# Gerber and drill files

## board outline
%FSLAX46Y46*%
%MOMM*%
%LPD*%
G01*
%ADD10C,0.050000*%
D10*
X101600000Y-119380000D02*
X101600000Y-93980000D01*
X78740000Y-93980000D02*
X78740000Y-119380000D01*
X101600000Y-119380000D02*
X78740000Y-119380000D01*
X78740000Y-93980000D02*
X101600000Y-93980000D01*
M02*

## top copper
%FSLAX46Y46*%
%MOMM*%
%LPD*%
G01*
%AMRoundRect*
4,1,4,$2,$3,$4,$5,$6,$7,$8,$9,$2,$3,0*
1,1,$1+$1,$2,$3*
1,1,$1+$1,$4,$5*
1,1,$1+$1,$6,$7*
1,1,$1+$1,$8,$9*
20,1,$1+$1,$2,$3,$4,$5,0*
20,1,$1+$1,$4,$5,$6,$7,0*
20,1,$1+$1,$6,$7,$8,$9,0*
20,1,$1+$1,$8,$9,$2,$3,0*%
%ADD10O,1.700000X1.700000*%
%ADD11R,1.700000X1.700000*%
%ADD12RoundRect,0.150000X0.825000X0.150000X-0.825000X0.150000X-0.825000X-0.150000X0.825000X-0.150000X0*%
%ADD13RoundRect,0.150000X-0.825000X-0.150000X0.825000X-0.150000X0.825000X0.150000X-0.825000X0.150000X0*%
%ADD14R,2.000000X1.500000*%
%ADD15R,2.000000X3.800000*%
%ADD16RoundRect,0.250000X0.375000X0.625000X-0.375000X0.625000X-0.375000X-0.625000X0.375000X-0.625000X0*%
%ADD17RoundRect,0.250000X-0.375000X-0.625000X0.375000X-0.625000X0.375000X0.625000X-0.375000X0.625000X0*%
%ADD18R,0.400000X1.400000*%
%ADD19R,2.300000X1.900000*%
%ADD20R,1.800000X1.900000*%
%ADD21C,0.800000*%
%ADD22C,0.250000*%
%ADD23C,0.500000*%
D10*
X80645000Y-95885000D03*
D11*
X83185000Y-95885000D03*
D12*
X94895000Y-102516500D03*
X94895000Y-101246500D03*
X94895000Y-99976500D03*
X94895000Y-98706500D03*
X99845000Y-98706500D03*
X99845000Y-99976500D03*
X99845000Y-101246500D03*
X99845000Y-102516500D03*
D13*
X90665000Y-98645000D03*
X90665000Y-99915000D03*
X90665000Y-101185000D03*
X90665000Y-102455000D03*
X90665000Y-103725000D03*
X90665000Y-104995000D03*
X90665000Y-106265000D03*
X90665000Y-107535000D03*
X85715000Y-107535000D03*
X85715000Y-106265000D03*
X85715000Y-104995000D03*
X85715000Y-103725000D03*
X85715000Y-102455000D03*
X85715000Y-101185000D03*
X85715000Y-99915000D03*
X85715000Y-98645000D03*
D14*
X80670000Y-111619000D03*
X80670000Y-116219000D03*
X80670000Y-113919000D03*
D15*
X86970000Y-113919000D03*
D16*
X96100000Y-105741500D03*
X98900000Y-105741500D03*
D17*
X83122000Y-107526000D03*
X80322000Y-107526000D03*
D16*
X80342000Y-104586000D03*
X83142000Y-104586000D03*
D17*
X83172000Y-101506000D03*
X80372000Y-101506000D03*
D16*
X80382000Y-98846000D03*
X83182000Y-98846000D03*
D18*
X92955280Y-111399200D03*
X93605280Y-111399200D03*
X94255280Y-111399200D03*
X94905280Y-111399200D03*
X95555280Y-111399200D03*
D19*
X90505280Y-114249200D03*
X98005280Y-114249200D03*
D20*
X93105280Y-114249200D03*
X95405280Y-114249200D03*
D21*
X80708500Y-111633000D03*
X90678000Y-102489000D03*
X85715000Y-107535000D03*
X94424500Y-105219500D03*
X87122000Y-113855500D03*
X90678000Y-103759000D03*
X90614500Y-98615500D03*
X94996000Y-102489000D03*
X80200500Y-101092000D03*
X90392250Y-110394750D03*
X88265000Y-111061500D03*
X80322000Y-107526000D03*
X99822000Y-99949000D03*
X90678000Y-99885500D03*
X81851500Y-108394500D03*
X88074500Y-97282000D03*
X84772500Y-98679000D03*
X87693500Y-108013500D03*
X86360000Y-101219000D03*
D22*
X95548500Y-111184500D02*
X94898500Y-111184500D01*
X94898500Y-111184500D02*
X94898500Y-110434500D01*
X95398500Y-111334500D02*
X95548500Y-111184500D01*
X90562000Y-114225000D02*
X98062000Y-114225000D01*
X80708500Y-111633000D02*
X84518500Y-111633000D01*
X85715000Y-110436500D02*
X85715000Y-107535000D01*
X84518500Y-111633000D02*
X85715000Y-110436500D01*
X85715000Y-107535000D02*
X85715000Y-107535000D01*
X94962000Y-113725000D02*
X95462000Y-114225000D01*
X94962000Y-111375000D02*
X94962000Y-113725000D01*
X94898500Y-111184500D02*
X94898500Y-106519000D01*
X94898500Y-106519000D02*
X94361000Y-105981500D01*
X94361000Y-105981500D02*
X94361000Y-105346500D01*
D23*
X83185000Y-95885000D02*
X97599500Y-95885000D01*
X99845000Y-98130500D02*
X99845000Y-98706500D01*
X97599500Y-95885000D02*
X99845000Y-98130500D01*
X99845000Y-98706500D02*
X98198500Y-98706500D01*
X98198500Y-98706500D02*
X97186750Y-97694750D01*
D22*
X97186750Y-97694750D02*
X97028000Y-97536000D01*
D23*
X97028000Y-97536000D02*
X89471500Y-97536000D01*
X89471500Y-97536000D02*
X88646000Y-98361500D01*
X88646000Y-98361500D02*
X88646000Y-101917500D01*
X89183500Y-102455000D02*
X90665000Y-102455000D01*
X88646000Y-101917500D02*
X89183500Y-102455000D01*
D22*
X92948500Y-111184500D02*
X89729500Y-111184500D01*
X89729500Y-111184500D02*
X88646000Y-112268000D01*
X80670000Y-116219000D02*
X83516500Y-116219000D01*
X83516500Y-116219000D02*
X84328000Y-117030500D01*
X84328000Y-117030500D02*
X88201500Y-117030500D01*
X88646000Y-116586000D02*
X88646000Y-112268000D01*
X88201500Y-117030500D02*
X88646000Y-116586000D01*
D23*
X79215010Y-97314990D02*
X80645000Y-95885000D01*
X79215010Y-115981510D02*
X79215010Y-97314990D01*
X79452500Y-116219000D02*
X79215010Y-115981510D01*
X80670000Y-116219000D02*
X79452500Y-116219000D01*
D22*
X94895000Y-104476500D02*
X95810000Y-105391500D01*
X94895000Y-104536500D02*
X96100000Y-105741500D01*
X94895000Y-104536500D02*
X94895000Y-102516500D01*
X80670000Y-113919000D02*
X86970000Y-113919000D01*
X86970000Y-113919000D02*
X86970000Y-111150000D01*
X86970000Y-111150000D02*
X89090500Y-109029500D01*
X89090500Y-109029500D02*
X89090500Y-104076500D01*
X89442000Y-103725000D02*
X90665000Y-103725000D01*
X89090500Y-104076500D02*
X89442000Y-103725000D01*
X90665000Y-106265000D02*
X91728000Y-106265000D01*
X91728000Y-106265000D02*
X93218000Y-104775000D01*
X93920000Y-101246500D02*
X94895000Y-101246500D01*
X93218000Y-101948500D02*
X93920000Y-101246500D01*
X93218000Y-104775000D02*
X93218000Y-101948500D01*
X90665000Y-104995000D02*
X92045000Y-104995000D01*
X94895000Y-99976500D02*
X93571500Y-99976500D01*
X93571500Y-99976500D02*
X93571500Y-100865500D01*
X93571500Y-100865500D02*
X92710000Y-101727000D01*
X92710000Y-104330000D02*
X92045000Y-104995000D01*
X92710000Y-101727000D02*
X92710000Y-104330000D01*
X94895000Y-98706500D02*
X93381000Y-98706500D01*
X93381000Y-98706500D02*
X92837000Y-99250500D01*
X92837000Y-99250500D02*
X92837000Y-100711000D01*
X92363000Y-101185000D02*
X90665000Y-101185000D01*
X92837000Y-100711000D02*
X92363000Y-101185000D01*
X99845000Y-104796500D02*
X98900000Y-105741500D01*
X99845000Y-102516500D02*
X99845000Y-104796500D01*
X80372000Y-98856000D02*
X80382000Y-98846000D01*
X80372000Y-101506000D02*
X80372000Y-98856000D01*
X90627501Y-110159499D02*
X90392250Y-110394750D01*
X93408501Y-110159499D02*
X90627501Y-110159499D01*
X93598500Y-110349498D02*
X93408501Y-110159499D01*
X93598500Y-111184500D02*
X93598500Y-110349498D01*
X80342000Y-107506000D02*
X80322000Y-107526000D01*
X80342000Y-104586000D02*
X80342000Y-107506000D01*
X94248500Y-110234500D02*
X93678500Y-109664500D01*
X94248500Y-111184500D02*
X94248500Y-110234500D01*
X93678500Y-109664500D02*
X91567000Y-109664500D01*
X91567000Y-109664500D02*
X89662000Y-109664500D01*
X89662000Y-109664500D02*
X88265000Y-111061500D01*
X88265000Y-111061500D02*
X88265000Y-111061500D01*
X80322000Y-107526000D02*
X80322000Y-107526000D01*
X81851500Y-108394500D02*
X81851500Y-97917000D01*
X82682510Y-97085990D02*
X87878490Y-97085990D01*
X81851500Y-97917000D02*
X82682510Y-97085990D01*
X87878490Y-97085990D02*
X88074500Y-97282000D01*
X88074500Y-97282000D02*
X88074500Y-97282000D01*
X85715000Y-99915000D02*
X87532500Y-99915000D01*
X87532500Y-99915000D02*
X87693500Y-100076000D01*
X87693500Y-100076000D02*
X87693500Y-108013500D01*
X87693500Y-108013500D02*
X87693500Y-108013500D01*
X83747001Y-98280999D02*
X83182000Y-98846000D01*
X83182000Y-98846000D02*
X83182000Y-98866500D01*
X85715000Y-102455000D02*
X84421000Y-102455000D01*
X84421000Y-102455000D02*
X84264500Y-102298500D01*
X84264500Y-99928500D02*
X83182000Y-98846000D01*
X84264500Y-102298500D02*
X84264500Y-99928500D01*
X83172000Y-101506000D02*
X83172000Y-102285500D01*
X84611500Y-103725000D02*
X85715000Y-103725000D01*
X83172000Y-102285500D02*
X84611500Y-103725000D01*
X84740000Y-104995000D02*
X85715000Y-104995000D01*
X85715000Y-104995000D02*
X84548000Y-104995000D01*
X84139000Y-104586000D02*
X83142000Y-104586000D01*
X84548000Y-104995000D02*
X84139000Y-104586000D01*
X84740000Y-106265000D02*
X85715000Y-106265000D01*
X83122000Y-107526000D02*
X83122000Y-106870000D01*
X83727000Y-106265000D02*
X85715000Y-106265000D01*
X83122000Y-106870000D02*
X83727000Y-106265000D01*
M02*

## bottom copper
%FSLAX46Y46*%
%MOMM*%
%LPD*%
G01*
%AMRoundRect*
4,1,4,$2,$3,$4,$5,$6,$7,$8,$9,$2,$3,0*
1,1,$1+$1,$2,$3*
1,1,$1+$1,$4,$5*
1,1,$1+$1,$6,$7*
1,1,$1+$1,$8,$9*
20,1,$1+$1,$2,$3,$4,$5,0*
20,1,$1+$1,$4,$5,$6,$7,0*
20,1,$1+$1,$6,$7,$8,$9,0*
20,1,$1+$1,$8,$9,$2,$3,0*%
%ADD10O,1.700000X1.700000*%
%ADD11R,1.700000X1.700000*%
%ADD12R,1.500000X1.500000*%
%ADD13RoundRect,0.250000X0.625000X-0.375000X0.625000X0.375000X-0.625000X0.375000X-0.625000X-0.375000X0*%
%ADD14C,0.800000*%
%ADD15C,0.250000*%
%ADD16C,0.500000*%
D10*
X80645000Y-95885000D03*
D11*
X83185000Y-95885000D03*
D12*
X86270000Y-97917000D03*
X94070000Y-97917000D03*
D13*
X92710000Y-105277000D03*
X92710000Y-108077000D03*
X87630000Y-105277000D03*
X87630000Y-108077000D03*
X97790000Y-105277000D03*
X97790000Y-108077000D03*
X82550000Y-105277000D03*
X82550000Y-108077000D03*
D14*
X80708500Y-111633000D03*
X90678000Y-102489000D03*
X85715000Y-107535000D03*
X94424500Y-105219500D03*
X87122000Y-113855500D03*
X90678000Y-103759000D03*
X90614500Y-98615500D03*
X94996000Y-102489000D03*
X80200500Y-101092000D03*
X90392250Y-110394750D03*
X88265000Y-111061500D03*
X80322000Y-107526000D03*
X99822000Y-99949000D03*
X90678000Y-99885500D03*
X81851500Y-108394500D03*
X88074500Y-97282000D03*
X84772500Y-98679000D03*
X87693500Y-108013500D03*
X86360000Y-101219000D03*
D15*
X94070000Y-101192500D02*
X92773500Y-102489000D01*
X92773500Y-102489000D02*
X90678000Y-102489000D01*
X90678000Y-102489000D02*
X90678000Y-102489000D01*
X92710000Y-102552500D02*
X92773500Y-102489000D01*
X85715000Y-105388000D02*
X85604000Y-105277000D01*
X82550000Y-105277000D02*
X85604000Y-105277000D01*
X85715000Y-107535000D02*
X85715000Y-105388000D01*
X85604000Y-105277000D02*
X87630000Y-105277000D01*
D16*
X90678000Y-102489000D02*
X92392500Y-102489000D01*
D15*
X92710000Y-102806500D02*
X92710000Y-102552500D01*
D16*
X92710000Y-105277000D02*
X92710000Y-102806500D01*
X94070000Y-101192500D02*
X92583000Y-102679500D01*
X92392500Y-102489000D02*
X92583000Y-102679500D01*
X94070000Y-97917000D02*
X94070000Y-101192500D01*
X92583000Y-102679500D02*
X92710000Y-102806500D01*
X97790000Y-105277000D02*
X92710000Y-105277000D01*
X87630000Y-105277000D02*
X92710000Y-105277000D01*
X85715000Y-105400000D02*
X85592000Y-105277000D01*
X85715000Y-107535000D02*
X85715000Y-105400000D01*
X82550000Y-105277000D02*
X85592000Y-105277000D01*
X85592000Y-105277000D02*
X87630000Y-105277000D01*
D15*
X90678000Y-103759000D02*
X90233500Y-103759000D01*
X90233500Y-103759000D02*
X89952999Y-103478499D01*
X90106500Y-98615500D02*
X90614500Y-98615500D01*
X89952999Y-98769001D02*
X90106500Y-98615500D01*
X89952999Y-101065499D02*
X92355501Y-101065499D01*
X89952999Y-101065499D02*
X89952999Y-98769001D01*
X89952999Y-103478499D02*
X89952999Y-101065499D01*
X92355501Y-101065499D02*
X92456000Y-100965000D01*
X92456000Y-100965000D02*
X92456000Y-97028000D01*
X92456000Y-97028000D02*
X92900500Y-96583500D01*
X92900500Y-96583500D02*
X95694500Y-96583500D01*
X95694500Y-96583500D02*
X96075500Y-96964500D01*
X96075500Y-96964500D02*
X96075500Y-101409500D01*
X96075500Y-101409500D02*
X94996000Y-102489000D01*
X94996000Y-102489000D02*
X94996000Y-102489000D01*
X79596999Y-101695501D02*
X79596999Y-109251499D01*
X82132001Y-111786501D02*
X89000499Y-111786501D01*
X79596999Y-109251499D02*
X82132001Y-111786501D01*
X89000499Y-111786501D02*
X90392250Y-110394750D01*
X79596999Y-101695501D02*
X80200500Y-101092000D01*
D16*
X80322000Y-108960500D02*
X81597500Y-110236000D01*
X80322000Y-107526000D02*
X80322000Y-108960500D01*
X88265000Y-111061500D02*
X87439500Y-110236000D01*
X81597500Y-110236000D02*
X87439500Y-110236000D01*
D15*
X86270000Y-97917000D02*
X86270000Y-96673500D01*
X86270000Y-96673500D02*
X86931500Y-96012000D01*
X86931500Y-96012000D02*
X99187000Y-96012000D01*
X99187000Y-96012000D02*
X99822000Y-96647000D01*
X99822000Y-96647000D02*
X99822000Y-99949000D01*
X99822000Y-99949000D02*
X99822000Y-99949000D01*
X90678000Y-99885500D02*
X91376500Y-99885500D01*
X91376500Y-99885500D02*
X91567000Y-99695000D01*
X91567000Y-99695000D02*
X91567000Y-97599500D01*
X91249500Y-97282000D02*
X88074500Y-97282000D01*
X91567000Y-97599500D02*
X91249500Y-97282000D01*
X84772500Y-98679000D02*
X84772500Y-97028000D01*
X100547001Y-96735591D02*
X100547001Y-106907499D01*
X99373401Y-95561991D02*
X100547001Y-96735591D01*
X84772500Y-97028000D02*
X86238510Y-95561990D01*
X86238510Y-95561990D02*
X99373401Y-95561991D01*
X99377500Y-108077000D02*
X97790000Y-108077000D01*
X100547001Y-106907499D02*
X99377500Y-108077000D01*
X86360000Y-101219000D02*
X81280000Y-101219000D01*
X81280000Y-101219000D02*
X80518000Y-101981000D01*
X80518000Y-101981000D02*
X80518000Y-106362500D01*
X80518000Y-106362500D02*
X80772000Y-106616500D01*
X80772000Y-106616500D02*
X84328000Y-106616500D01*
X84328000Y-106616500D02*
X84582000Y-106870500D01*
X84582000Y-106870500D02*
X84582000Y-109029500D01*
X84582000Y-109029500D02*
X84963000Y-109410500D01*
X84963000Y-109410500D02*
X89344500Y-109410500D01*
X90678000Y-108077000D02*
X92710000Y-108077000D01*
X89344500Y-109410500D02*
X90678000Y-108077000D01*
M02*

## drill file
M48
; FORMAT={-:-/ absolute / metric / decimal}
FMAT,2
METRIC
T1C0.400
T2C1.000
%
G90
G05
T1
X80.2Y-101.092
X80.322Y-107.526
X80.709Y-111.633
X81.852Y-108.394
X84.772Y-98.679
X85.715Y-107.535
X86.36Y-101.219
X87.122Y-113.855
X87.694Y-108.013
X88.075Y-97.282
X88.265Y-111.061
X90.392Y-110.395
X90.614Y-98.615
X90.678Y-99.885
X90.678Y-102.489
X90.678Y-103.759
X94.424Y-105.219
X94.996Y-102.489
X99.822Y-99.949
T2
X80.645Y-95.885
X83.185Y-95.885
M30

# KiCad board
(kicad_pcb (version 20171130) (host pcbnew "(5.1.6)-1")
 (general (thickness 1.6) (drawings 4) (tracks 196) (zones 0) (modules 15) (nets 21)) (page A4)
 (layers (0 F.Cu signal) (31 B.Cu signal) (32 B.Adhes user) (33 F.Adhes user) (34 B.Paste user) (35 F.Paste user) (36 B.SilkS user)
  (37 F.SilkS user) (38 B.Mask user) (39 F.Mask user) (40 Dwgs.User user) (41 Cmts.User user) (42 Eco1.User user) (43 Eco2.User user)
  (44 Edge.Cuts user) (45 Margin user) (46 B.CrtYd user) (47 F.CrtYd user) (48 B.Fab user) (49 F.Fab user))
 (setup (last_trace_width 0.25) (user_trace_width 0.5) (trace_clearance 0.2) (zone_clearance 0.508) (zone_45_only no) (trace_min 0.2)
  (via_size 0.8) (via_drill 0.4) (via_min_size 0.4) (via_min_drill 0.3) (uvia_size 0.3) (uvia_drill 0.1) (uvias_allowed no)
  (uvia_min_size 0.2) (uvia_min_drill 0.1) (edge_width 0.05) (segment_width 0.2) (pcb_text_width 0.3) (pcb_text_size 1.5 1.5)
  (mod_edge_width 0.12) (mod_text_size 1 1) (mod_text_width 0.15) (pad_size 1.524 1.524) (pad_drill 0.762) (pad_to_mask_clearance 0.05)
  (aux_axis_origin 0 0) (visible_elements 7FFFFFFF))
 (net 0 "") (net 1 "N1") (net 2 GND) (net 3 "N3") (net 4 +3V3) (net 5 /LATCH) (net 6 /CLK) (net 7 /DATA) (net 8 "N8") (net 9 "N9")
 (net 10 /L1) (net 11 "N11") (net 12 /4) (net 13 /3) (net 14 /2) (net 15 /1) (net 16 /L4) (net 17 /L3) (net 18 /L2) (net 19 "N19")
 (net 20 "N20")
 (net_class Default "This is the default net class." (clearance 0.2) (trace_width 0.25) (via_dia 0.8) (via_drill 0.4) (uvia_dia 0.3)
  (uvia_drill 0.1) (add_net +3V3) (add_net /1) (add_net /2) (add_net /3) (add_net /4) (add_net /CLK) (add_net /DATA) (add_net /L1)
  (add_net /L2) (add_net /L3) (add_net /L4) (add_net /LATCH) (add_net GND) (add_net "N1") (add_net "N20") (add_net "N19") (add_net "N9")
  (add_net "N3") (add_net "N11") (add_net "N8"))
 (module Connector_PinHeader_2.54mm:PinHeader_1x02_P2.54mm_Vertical (layer F.Cu) (at 83.185 95.885 270)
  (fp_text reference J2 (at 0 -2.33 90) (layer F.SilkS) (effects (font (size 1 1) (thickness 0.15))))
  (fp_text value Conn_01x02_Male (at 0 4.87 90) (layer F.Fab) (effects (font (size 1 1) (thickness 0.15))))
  (pad 2 thru_hole oval (at 0 2.54 270) (size 1.7 1.7) (drill 1) (layers *.Cu *.Mask) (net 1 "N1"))
  (pad 1 thru_hole rect (at 0 0 270) (size 1.7 1.7) (drill 1) (layers *.Cu *.Mask) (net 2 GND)))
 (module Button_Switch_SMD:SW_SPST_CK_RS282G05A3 (layer B.Cu) (at 90.17 97.917 180)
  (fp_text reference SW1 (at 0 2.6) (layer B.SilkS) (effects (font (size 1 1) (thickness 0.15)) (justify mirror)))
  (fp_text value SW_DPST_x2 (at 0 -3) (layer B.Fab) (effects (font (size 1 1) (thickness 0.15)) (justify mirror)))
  (pad 2 smd rect (at 3.9 0 180) (size 1.5 1.5) (layers B.Cu B.Paste B.Mask) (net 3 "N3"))
  (pad 1 smd rect (at -3.9 0 180) (size 1.5 1.5) (layers B.Cu B.Paste B.Mask) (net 2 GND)))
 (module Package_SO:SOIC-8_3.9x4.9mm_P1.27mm (layer F.Cu) (at 97.37 100.6115 180)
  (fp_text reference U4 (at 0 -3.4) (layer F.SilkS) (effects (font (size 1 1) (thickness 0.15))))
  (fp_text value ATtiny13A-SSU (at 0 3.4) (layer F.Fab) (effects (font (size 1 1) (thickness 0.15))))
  (pad 8 smd roundrect (at 2.475 -1.905 180) (size 1.95 0.6) (layers F.Cu F.Paste F.Mask) (roundrect_rratio 0.25) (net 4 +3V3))
  (pad 7 smd roundrect (at 2.475 -0.635 180) (size 1.95 0.6) (layers F.Cu F.Paste F.Mask) (roundrect_rratio 0.25) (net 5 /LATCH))
  (pad 6 smd roundrect (at 2.475 0.635 180) (size 1.95 0.6) (layers F.Cu F.Paste F.Mask) (roundrect_rratio 0.25) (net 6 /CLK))
  (pad 5 smd roundrect (at 2.475 1.905 180) (size 1.95 0.6) (layers F.Cu F.Paste F.Mask) (roundrect_rratio 0.25) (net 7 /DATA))
  (pad 4 smd roundrect (at -2.475 1.905 180) (size 1.95 0.6) (layers F.Cu F.Paste F.Mask) (roundrect_rratio 0.25) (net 2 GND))
  (pad 3 smd roundrect (at -2.475 0.635 180) (size 1.95 0.6) (layers F.Cu F.Paste F.Mask) (roundrect_rratio 0.25) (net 3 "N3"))
  (pad 2 smd roundrect (at -2.475 -0.635 180) (size 1.95 0.6) (layers F.Cu F.Paste F.Mask) (roundrect_rratio 0.25) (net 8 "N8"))
  (pad 1 smd roundrect (at -2.475 -1.905 180) (size 1.95 0.6) (layers F.Cu F.Paste F.Mask) (roundrect_rratio 0.25) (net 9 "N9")))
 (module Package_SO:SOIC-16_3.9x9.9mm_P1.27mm (layer F.Cu) (at 88.19 103.09)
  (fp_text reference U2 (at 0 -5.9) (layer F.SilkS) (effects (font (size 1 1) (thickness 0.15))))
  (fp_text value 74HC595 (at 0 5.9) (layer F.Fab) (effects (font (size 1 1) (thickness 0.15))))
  (pad 16 smd roundrect (at 2.475 -4.445) (size 1.95 0.6) (layers F.Cu F.Paste F.Mask) (roundrect_rratio 0.25) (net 4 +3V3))
  (pad 15 smd roundrect (at 2.475 -3.175) (size 1.95 0.6) (layers F.Cu F.Paste F.Mask) (roundrect_rratio 0.25) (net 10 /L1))
  (pad 14 smd roundrect (at 2.475 -1.905) (size 1.95 0.6) (layers F.Cu F.Paste F.Mask) (roundrect_rratio 0.25) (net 7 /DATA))
  (pad 13 smd roundrect (at 2.475 -0.635) (size 1.95 0.6) (layers F.Cu F.Paste F.Mask) (roundrect_rratio 0.25) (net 2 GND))
  (pad 12 smd roundrect (at 2.475 0.635) (size 1.95 0.6) (layers F.Cu F.Paste F.Mask) (roundrect_rratio 0.25) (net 4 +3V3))
  (pad 11 smd roundrect (at 2.475 1.905) (size 1.95 0.6) (layers F.Cu F.Paste F.Mask) (roundrect_rratio 0.25) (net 6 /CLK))
  (pad 10 smd roundrect (at 2.475 3.175) (size 1.95 0.6) (layers F.Cu F.Paste F.Mask) (roundrect_rratio 0.25) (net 5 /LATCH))
  (pad 9 smd roundrect (at 2.475 4.445) (size 1.95 0.6) (layers F.Cu F.Paste F.Mask) (roundrect_rratio 0.25) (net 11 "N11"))
  (pad 8 smd roundrect (at -2.475 4.445) (size 1.95 0.6) (layers F.Cu F.Paste F.Mask) (roundrect_rratio 0.25) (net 2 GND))
  (pad 7 smd roundrect (at -2.475 3.175) (size 1.95 0.6) (layers F.Cu F.Paste F.Mask) (roundrect_rratio 0.25) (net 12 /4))
  (pad 6 smd roundrect (at -2.475 1.905) (size 1.95 0.6) (layers F.Cu F.Paste F.Mask) (roundrect_rratio 0.25) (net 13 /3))
  (pad 5 smd roundrect (at -2.475 0.635) (size 1.95 0.6) (layers F.Cu F.Paste F.Mask) (roundrect_rratio 0.25) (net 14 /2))
  (pad 4 smd roundrect (at -2.475 -0.635) (size 1.95 0.6) (layers F.Cu F.Paste F.Mask) (roundrect_rratio 0.25) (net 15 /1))
  (pad 3 smd roundrect (at -2.475 -1.905) (size 1.95 0.6) (layers F.Cu F.Paste F.Mask) (roundrect_rratio 0.25) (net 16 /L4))
  (pad 2 smd roundrect (at -2.475 -3.175) (size 1.95 0.6) (layers F.Cu F.Paste F.Mask) (roundrect_rratio 0.25) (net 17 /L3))
  (pad 1 smd roundrect (at -2.475 -4.445) (size 1.95 0.6) (layers F.Cu F.Paste F.Mask) (roundrect_rratio 0.25) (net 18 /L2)))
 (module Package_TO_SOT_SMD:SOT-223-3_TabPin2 (layer F.Cu) (at 83.82 113.919)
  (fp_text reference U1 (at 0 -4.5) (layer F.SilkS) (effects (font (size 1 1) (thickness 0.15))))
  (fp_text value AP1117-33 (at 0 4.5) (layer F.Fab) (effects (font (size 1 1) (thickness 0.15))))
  (pad 1 smd rect (at -3.15 -2.3) (size 2 1.5) (layers F.Cu F.Paste F.Mask) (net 2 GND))
  (pad 3 smd rect (at -3.15 2.3) (size 2 1.5) (layers F.Cu F.Paste F.Mask) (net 1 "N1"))
  (pad 2 smd rect (at -3.15 0) (size 2 1.5) (layers F.Cu F.Paste F.Mask) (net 4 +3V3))
  (pad 2 smd rect (at 3.15 0) (size 2 3.8) (layers F.Cu F.Paste F.Mask) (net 4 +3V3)))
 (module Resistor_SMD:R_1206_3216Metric (layer F.Cu) (at 97.5 105.7415 180)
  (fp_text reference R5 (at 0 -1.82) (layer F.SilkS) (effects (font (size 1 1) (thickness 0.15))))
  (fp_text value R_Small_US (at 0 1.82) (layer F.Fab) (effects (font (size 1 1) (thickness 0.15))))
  (pad 2 smd roundrect (at 1.4 0 180) (size 1.25 1.75) (layers F.Cu F.Paste F.Mask) (roundrect_rratio 0.2) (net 4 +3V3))
  (pad 1 smd roundrect (at -1.4 0 180) (size 1.25 1.75) (layers F.Cu F.Paste F.Mask) (roundrect_rratio 0.2) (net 9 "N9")))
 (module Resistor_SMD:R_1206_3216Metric (layer F.Cu) (at 81.722 107.526)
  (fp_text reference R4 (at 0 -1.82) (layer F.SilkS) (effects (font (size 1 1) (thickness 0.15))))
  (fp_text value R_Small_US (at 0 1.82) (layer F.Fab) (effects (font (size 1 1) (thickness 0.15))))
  (pad 2 smd roundrect (at 1.4 0) (size 1.25 1.75) (layers F.Cu F.Paste F.Mask) (roundrect_rratio 0.2) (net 12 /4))
  (pad 1 smd roundrect (at -1.4 0) (size 1.25 1.75) (layers F.Cu F.Paste F.Mask) (roundrect_rratio 0.2) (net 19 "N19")))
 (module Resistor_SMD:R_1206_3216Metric (layer F.Cu) (at 81.742 104.586 180)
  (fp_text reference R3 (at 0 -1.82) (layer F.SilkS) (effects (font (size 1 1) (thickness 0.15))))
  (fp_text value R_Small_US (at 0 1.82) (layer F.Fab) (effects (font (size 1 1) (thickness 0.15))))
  (pad 2 smd roundrect (at 1.4 0 180) (size 1.25 1.75) (layers F.Cu F.Paste F.Mask) (roundrect_rratio 0.2) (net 19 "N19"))
  (pad 1 smd roundrect (at -1.4 0 180) (size 1.25 1.75) (layers F.Cu F.Paste F.Mask) (roundrect_rratio 0.2) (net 13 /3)))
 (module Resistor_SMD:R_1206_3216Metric (layer F.Cu) (at 81.772 101.506)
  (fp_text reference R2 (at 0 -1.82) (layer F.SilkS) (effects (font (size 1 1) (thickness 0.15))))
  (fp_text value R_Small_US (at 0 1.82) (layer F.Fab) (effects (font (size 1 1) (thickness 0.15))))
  (pad 2 smd roundrect (at 1.4 0) (size 1.25 1.75) (layers F.Cu F.Paste F.Mask) (roundrect_rratio 0.2) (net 14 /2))
  (pad 1 smd roundrect (at -1.4 0) (size 1.25 1.75) (layers F.Cu F.Paste F.Mask) (roundrect_rratio 0.2) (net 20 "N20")))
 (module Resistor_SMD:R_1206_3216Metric (layer F.Cu) (at 81.782 98.846 180)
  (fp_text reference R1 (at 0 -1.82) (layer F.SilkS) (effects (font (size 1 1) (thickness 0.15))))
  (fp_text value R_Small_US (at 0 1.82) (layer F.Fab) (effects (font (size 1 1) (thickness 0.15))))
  (pad 2 smd roundrect (at 1.4 0 180) (size 1.25 1.75) (layers F.Cu F.Paste F.Mask) (roundrect_rratio 0.2) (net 20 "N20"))
  (pad 1 smd roundrect (at -1.4 0 180) (size 1.25 1.75) (layers F.Cu F.Paste F.Mask) (roundrect_rratio 0.2) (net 15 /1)))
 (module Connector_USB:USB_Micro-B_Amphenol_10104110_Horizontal (layer F.Cu) (at 94.25528 112.9492)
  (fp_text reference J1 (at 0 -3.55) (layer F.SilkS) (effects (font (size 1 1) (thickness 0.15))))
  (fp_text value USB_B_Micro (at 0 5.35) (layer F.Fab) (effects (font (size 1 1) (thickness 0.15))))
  (pad 1 smd rect (at -1.3 -1.55) (size 0.4 1.4) (layers F.Cu F.Paste F.Mask) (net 1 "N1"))
  (pad 2 smd rect (at -0.65 -1.55) (size 0.4 1.4) (layers F.Cu F.Paste F.Mask) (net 20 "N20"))
  (pad 3 smd rect (at 0 -1.55) (size 0.4 1.4) (layers F.Cu F.Paste F.Mask) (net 19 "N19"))
  (pad 4 smd rect (at 0.65 -1.55) (size 0.4 1.4) (layers F.Cu F.Paste F.Mask) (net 2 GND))
  (pad 5 smd rect (at 1.3 -1.55) (size 0.4 1.4) (layers F.Cu F.Paste F.Mask) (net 2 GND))
  (pad 6 smd rect (at -3.75 1.3) (size 2.3 1.9) (layers F.Cu F.Paste F.Mask) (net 2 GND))
  (pad 6 smd rect (at 3.75 1.3) (size 2.3 1.9) (layers F.Cu F.Paste F.Mask) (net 2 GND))
  (pad 6 smd rect (at -1.15 1.3) (size 1.8 1.9) (layers F.Cu F.Paste F.Mask) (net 2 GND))
  (pad 6 smd rect (at 1.15 1.3) (size 1.8 1.9) (layers F.Cu F.Paste F.Mask) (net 2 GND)))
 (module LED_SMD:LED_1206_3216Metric (layer B.Cu) (at 92.71 106.677 90)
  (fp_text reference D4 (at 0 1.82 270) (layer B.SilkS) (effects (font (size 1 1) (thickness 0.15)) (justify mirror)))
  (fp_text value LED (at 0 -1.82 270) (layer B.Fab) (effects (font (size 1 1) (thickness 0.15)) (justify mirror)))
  (pad 2 smd roundrect (at 1.4 0 90) (size 1.25 1.75) (layers B.Cu B.Paste B.Mask) (roundrect_rratio 0.2) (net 2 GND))
  (pad 1 smd roundrect (at -1.4 0 90) (size 1.25 1.75) (layers B.Cu B.Paste B.Mask) (roundrect_rratio 0.2) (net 16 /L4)))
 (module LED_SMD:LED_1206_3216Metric (layer B.Cu) (at 87.63 106.677 90)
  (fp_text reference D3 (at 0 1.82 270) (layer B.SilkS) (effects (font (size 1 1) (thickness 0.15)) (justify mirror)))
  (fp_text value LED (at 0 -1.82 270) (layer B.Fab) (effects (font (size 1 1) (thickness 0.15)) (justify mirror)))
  (pad 2 smd roundrect (at 1.4 0 90) (size 1.25 1.75) (layers B.Cu B.Paste B.Mask) (roundrect_rratio 0.2) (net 2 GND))
  (pad 1 smd roundrect (at -1.4 0 90) (size 1.25 1.75) (layers B.Cu B.Paste B.Mask) (roundrect_rratio 0.2) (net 17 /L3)))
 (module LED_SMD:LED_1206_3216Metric (layer B.Cu) (at 97.79 106.677 90)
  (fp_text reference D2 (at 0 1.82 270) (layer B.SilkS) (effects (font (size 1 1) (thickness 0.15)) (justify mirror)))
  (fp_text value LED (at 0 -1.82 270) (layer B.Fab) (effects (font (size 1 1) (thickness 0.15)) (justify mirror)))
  (pad 2 smd roundrect (at 1.4 0 90) (size 1.25 1.75) (layers B.Cu B.Paste B.Mask) (roundrect_rratio 0.2) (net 2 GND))
  (pad 1 smd roundrect (at -1.4 0 90) (size 1.25 1.75) (layers B.Cu B.Paste B.Mask) (roundrect_rratio 0.2) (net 18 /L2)))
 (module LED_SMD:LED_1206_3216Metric (layer B.Cu) (at 82.55 106.677 90)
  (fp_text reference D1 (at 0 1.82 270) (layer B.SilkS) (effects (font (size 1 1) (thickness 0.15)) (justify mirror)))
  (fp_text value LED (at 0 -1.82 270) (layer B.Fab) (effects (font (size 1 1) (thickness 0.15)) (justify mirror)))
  (pad 2 smd roundrect (at 1.4 0 90) (size 1.25 1.75) (layers B.Cu B.Paste B.Mask) (roundrect_rratio 0.2) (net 2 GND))
  (pad 1 smd roundrect (at -1.4 0 90) (size 1.25 1.75) (layers B.Cu B.Paste B.Mask) (roundrect_rratio 0.2) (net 10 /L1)))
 (gr_line (start 101.6 119.38) (end 101.6 93.98) (layer Edge.Cuts) (width 0.05))
 (gr_line (start 78.74 93.98) (end 78.74 119.38) (layer Edge.Cuts) (width 0.05))
 (gr_line (start 101.6 119.38) (end 78.74 119.38) (layer Edge.Cuts) (width 0.05))
 (gr_line (start 78.74 93.98) (end 101.6 93.98) (layer Edge.Cuts) (width 0.05))
 (via (at 80.7085 111.633) (size 0.8) (drill 0.4) (layers F.Cu B.Cu) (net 2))
 (segment (start 95.5485 111.1845) (end 94.8985 111.1845) (width 0.25) (layer F.Cu) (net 2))
 (segment (start 94.8985 111.1845) (end 94.8985 110.4345) (width 0.25) (layer F.Cu) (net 2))
 (segment (start 95.3985 111.3345) (end 95.5485 111.1845) (width 0.25) (layer F.Cu) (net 2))
 (segment (start 90.562 114.225) (end 98.062 114.225) (width 0.25) (layer F.Cu) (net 2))
 (segment (start 94.07 101.1925) (end 92.7735 102.489) (width 0.25) (layer B.Cu) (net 2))
 (segment (start 92.7735 102.489) (end 90.678 102.489) (width 0.25) (layer B.Cu) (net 2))
 (segment (start 90.678 102.489) (end 90.678 102.489) (width 0.25) (layer B.Cu) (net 2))
 (via (at 90.678 102.489) (size 0.8) (drill 0.4) (layers F.Cu B.Cu) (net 2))
 (segment (start 92.71 102.5525) (end 92.7735 102.489) (width 0.25) (layer B.Cu) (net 2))
 (segment (start 80.7085 111.633) (end 84.5185 111.633) (width 0.25) (layer F.Cu) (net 2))
 (segment (start 85.715 110.4365) (end 85.715 107.535) (width 0.25) (layer F.Cu) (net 2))
 (segment (start 84.5185 111.633) (end 85.715 110.4365) (width 0.25) (layer F.Cu) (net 2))
 (segment (start 85.715 107.535) (end 85.715 107.535) (width 0.25) (layer F.Cu) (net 2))
 (via (at 85.715 107.535) (size 0.8) (drill 0.4) (layers F.Cu B.Cu) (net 2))
 (segment (start 85.715 105.388) (end 85.604 105.277) (width 0.25) (layer B.Cu) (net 2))
 (segment (start 82.55 105.277) (end 85.604 105.277) (width 0.25) (layer B.Cu) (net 2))
 (segment (start 85.715 107.535) (end 85.715 105.388) (width 0.25) (layer B.Cu) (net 2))
 (segment (start 85.604 105.277) (end 87.63 105.277) (width 0.25) (layer B.Cu) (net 2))
 (segment (start 94.962 113.725) (end 95.462 114.225) (width 0.25) (layer F.Cu) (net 2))
 (segment (start 94.962 111.375) (end 94.962 113.725) (width 0.25) (layer F.Cu) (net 2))
 (segment (start 94.8985 111.1845) (end 94.8985 106.519) (width 0.25) (layer F.Cu) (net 2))
 (segment (start 94.8985 106.519) (end 94.361 105.9815) (width 0.25) (layer F.Cu) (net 2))
 (segment (start 94.361 105.9815) (end 94.361 105.3465) (width 0.25) (layer F.Cu) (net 2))
 (via (at 94.4245 105.2195) (size 0.8) (drill 0.4) (layers F.Cu B.Cu) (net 2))
 (segment (start 83.185 95.885) (end 97.5995 95.885) (width 0.5) (layer F.Cu) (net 2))
 (segment (start 99.845 98.1305) (end 99.845 98.7065) (width 0.5) (layer F.Cu) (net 2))
 (segment (start 97.5995 95.885) (end 99.845 98.1305) (width 0.5) (layer F.Cu) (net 2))
 (segment (start 99.845 98.7065) (end 98.1985 98.7065) (width 0.5) (layer F.Cu) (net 2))
 (segment (start 98.1985 98.7065) (end 97.18675 97.69475) (width 0.5) (layer F.Cu) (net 2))
 (segment (start 97.18675 97.69475) (end 97.028 97.536) (width 0.25) (layer F.Cu) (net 2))
 (segment (start 97.028 97.536) (end 89.4715 97.536) (width 0.5) (layer F.Cu) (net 2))
 (segment (start 89.4715 97.536) (end 88.646 98.3615) (width 0.5) (layer F.Cu) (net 2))
 (segment (start 88.646 98.3615) (end 88.646 101.9175) (width 0.5) (layer F.Cu) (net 2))
 (segment (start 89.1835 102.455) (end 90.665 102.455) (width 0.5) (layer F.Cu) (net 2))
 (segment (start 88.646 101.9175) (end 89.1835 102.455) (width 0.5) (layer F.Cu) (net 2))
 (segment (start 90.678 102.489) (end 92.3925 102.489) (width 0.5) (layer B.Cu) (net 2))
 (segment (start 92.71 102.8065) (end 92.71 102.5525) (width 0.25) (layer B.Cu) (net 2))
 (segment (start 92.71 105.277) (end 92.71 102.8065) (width 0.5) (layer B.Cu) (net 2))
 (segment (start 94.07 101.1925) (end 92.583 102.6795) (width 0.5) (layer B.Cu) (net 2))
 (segment (start 92.3925 102.489) (end 92.583 102.6795) (width 0.5) (layer B.Cu) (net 2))
 (segment (start 94.07 97.917) (end 94.07 101.1925) (width 0.5) (layer B.Cu) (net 2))
 (segment (start 92.583 102.6795) (end 92.71 102.8065) (width 0.5) (layer B.Cu) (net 2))
 (segment (start 97.79 105.277) (end 92.71 105.277) (width 0.5) (layer B.Cu) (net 2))
 (segment (start 87.63 105.277) (end 92.71 105.277) (width 0.5) (layer B.Cu) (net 2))
 (segment (start 85.715 105.4) (end 85.592 105.277) (width 0.5) (layer B.Cu) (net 2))
 (segment (start 85.715 107.535) (end 85.715 105.4) (width 0.5) (layer B.Cu) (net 2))
 (segment (start 82.55 105.277) (end 85.592 105.277) (width 0.5) (layer B.Cu) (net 2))
 (segment (start 85.592 105.277) (end 87.63 105.277) (width 0.5) (layer B.Cu) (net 2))
 (segment (start 92.9485 111.1845) (end 89.7295 111.1845) (width 0.25) (layer F.Cu) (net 1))
 (segment (start 89.7295 111.1845) (end 88.646 112.268) (width 0.25) (layer F.Cu) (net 1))
 (segment (start 80.67 116.219) (end 83.5165 116.219) (width 0.25) (layer F.Cu) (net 1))
 (segment (start 83.5165 116.219) (end 84.328 117.0305) (width 0.25) (layer F.Cu) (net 1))
 (segment (start 84.328 117.0305) (end 88.2015 117.0305) (width 0.25) (layer F.Cu) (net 1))
 (segment (start 88.646 116.586) (end 88.646 112.268) (width 0.25) (layer F.Cu) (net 1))
 (segment (start 88.2015 117.0305) (end 88.646 116.586) (width 0.25) (layer F.Cu) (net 1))
 (segment (start 79.21501 97.31499) (end 80.645 95.885) (width 0.5) (layer F.Cu) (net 1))
 (segment (start 79.21501 115.98151) (end 79.21501 97.31499) (width 0.5) (layer F.Cu) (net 1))
 (segment (start 79.4525 116.219) (end 79.21501 115.98151) (width 0.5) (layer F.Cu) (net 1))
 (segment (start 80.67 116.219) (end 79.4525 116.219) (width 0.5) (layer F.Cu) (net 1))
 (via (at 87.122 113.8555) (size 0.8) (drill 0.4) (layers F.Cu B.Cu) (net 4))
 (via (at 90.678 103.759) (size 0.8) (drill 0.4) (layers F.Cu B.Cu) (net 4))
 (via (at 90.6145 98.6155) (size 0.8) (drill 0.4) (layers F.Cu B.Cu) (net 4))
 (segment (start 94.895 104.4765) (end 95.81 105.3915) (width 0.25) (layer F.Cu) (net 4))
 (segment (start 94.895 104.5365) (end 96.1 105.7415) (width 0.25) (layer F.Cu) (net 4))
 (segment (start 94.895 104.5365) (end 94.895 102.5165) (width 0.25) (layer F.Cu) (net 4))
 (segment (start 90.678 103.759) (end 90.2335 103.759) (width 0.25) (layer B.Cu) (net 4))
 (segment (start 90.2335 103.759) (end 89.952999 103.478499) (width 0.25) (layer B.Cu) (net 4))
 (segment (start 90.1065 98.6155) (end 90.6145 98.6155) (width 0.25) (layer B.Cu) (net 4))
 (segment (start 89.952999 98.769001) (end 90.1065 98.6155) (width 0.25) (layer B.Cu) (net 4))
 (segment (start 80.67 113.919) (end 86.97 113.919) (width 0.25) (layer F.Cu) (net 4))
 (segment (start 86.97 113.919) (end 86.97 111.15) (width 0.25) (layer F.Cu) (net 4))
 (segment (start 86.97 111.15) (end 89.0905 109.0295) (width 0.25) (layer F.Cu) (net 4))
 (segment (start 89.0905 109.0295) (end 89.0905 104.0765) (width 0.25) (layer F.Cu) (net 4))
 (segment (start 89.442 103.725) (end 90.665 103.725) (width 0.25) (layer F.Cu) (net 4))
 (segment (start 89.0905 104.0765) (end 89.442 103.725) (width 0.25) (layer F.Cu) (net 4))
 (segment (start 89.952999 101.065499) (end 92.355501 101.065499) (width 0.25) (layer B.Cu) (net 4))
 (segment (start 89.952999 101.065499) (end 89.952999 98.769001) (width 0.25) (layer B.Cu) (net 4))
 (segment (start 89.952999 103.478499) (end 89.952999 101.065499) (width 0.25) (layer B.Cu) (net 4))
 (segment (start 92.355501 101.065499) (end 92.456 100.965) (width 0.25) (layer B.Cu) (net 4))
 (segment (start 92.456 100.965) (end 92.456 97.028) (width 0.25) (layer B.Cu) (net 4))
 (segment (start 92.456 97.028) (end 92.9005 96.5835) (width 0.25) (layer B.Cu) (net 4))
 (segment (start 92.9005 96.5835) (end 95.6945 96.5835) (width 0.25) (layer B.Cu) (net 4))
 (segment (start 95.6945 96.5835) (end 96.0755 96.9645) (width 0.25) (layer B.Cu) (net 4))
 (segment (start 96.0755 96.9645) (end 96.0755 101.4095) (width 0.25) (layer B.Cu) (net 4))
 (segment (start 96.0755 101.4095) (end 94.996 102.489) (width 0.25) (layer B.Cu) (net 4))
 (segment (start 94.996 102.489) (end 94.996 102.489) (width 0.25) (layer B.Cu) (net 4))
 (via (at 94.996 102.489) (size 0.8) (drill 0.4) (layers F.Cu B.Cu) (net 4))
 (segment (start 90.665 106.265) (end 91.728 106.265) (width 0.25) (layer F.Cu) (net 5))
 (segment (start 91.728 106.265) (end 93.218 104.775) (width 0.25) (layer F.Cu) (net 5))
 (segment (start 93.92 101.2465) (end 94.895 101.2465) (width 0.25) (layer F.Cu) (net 5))
 (segment (start 93.218 101.9485) (end 93.92 101.2465) (width 0.25) (layer F.Cu) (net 5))
 (segment (start 93.218 104.775) (end 93.218 101.9485) (width 0.25) (layer F.Cu) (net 5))
 (segment (start 90.665 104.995) (end 92.045 104.995) (width 0.25) (layer F.Cu) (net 6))
 (segment (start 94.895 99.9765) (end 93.5715 99.9765) (width 0.25) (layer F.Cu) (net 6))
 (segment (start 93.5715 99.9765) (end 93.5715 100.8655) (width 0.25) (layer F.Cu) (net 6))
 (segment (start 93.5715 100.8655) (end 92.71 101.727) (width 0.25) (layer F.Cu) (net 6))
 (segment (start 92.71 104.33) (end 92.045 104.995) (width 0.25) (layer F.Cu) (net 6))
 (segment (start 92.71 101.727) (end 92.71 104.33) (width 0.25) (layer F.Cu) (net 6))
 (segment (start 94.895 98.7065) (end 93.381 98.7065) (width 0.25) (layer F.Cu) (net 7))
 (segment (start 93.381 98.7065) (end 92.837 99.2505) (width 0.25) (layer F.Cu) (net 7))
 (segment (start 92.837 99.2505) (end 92.837 100.711) (width 0.25) (layer F.Cu) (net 7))
 (segment (start 92.363 101.185) (end 90.665 101.185) (width 0.25) (layer F.Cu) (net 7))
 (segment (start 92.837 100.711) (end 92.363 101.185) (width 0.25) (layer F.Cu) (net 7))
 (segment (start 99.845 104.7965) (end 98.9 105.7415) (width 0.25) (layer F.Cu) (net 9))
 (segment (start 99.845 102.5165) (end 99.845 104.7965) (width 0.25) (layer F.Cu) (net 9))
 (via (at 80.2005 101.092) (size 0.8) (drill 0.4) (layers F.Cu B.Cu) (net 20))
 (segment (start 80.372 98.856) (end 80.382 98.846) (width 0.25) (layer F.Cu) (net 20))
 (segment (start 80.372 101.506) (end 80.372 98.856) (width 0.25) (layer F.Cu) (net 20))
 (segment (start 79.596999 101.695501) (end 79.596999 109.251499) (width 0.25) (layer B.Cu) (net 20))
 (segment (start 82.132001 111.786501) (end 89.000499 111.786501) (width 0.25) (layer B.Cu) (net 20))
 (segment (start 79.596999 109.251499) (end 82.132001 111.786501) (width 0.25) (layer B.Cu) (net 20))
 (segment (start 89.000499 111.786501) (end 90.39225 110.39475) (width 0.25) (layer B.Cu) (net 20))
 (via (at 90.39225 110.39475) (size 0.8) (drill 0.4) (layers F.Cu B.Cu) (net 20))
 (segment (start 90.627501 110.159499) (end 90.39225 110.39475) (width 0.25) (layer F.Cu) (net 20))
 (segment (start 93.408501 110.159499) (end 90.627501 110.159499) (width 0.25) (layer F.Cu) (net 20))
 (segment (start 93.5985 110.349498) (end 93.408501 110.159499) (width 0.25) (layer F.Cu) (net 20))
 (segment (start 93.5985 111.1845) (end 93.5985 110.349498) (width 0.25) (layer F.Cu) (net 20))
 (segment (start 79.596999 101.695501) (end 80.2005 101.092) (width 0.25) (layer B.Cu) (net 20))
 (segment (start 80.342 107.506) (end 80.322 107.526) (width 0.25) (layer F.Cu) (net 19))
 (segment (start 80.342 104.586) (end 80.342 107.506) (width 0.25) (layer F.Cu) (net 19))
 (segment (start 94.2485 110.2345) (end 93.6785 109.6645) (width 0.25) (layer F.Cu) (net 19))
 (segment (start 94.2485 111.1845) (end 94.2485 110.2345) (width 0.25) (layer F.Cu) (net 19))
 (segment (start 93.6785 109.6645) (end 91.567 109.6645) (width 0.25) (layer F.Cu) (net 19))
 (segment (start 91.567 109.6645) (end 89.662 109.6645) (width 0.25) (layer F.Cu) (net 19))
 (segment (start 89.662 109.6645) (end 88.265 111.0615) (width 0.25) (layer F.Cu) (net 19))
 (segment (start 88.265 111.0615) (end 88.265 111.0615) (width 0.25) (layer F.Cu) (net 19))
 (via (at 88.265 111.0615) (size 0.8) (drill 0.4) (layers F.Cu B.Cu) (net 19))
 (segment (start 80.322 107.526) (end 80.322 107.526) (width 0.25) (layer F.Cu) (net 19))
 (via (at 80.322 107.526) (size 0.8) (drill 0.4) (layers F.Cu B.Cu) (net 19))
 (segment (start 80.322 108.9605) (end 81.5975 110.236) (width 0.5) (layer B.Cu) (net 19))
 (segment (start 80.322 107.526) (end 80.322 108.9605) (width 0.5) (layer B.Cu) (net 19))
 (segment (start 88.265 111.0615) (end 87.4395 110.236) (width 0.5) (layer B.Cu) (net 19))
 (segment (start 81.5975 110.236) (end 87.4395 110.236) (width 0.5) (layer B.Cu) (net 19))
 (segment (start 86.27 97.917) (end 86.27 96.6735) (width 0.25) (layer B.Cu) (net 3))
 (segment (start 86.27 96.6735) (end 86.9315 96.012) (width 0.25) (layer B.Cu) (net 3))
 (segment (start 86.9315 96.012) (end 99.187 96.012) (width 0.25) (layer B.Cu) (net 3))
 (segment (start 99.187 96.012) (end 99.822 96.647) (width 0.25) (layer B.Cu) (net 3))
 (segment (start 99.822 96.647) (end 99.822 99.949) (width 0.25) (layer B.Cu) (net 3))
 (segment (start 99.822 99.949) (end 99.822 99.949) (width 0.25) (layer B.Cu) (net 3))
 (via (at 99.822 99.949) (size 0.8) (drill 0.4) (layers F.Cu B.Cu) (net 3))
 (via (at 90.678 99.8855) (size 0.8) (drill 0.4) (layers F.Cu B.Cu) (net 10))
 (via (at 81.8515 108.3945) (size 0.8) (drill 0.4) (layers F.Cu B.Cu) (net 10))
 (segment (start 81.8515 108.3945) (end 81.8515 97.917) (width 0.25) (layer F.Cu) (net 10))
 (segment (start 82.68251 97.08599) (end 87.87849 97.08599) (width 0.25) (layer F.Cu) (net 10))
 (segment (start 81.8515 97.917) (end 82.68251 97.08599) (width 0.25) (layer F.Cu) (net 10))
 (segment (start 87.87849 97.08599) (end 88.0745 97.282) (width 0.25) (layer F.Cu) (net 10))
 (segment (start 88.0745 97.282) (end 88.0745 97.282) (width 0.25) (layer F.Cu) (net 10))
 (via (at 88.0745 97.282) (size 0.8) (drill 0.4) (layers F.Cu B.Cu) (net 10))
 (segment (start 90.678 99.8855) (end 91.3765 99.8855) (width 0.25) (layer B.Cu) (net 10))
 (segment (start 91.3765 99.8855) (end 91.567 99.695) (width 0.25) (layer B.Cu) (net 10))
 (segment (start 91.567 99.695) (end 91.567 97.5995) (width 0.25) (layer B.Cu) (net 10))
 (segment (start 91.2495 97.282) (end 88.0745 97.282) (width 0.25) (layer B.Cu) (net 10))
 (segment (start 91.567 97.5995) (end 91.2495 97.282) (width 0.25) (layer B.Cu) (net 10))
 (via (at 84.7725 98.679) (size 0.8) (drill 0.4) (layers F.Cu B.Cu) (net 18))
 (segment (start 84.7725 98.679) (end 84.7725 97.028) (width 0.25) (layer B.Cu) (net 18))
 (segment (start 100.547001 96.735591) (end 100.547001 106.907499) (width 0.25) (layer B.Cu) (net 18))
 (segment (start 99.373401 95.561991) (end 100.547001 96.735591) (width 0.25) (layer B.Cu) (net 18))
 (segment (start 84.7725 97.028) (end 86.23851 95.56199) (width 0.25) (layer B.Cu) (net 18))
 (segment (start 86.23851 95.56199) (end 99.373401 95.561991) (width 0.25) (layer B.Cu) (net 18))
 (segment (start 99.3775 108.077) (end 97.79 108.077) (width 0.25) (layer B.Cu) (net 18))
 (segment (start 100.547001 106.907499) (end 99.3775 108.077) (width 0.25) (layer B.Cu) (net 18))
 (segment (start 85.715 99.915) (end 87.5325 99.915) (width 0.25) (layer F.Cu) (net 17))
 (segment (start 87.5325 99.915) (end 87.6935 100.076) (width 0.25) (layer F.Cu) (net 17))
 (segment (start 87.6935 100.076) (end 87.6935 108.0135) (width 0.25) (layer F.Cu) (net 17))
 (segment (start 87.6935 108.0135) (end 87.6935 108.0135) (width 0.25) (layer F.Cu) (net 17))
 (via (at 87.6935 108.0135) (size 0.8) (drill 0.4) (layers F.Cu B.Cu) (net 17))
 (via (at 86.36 101.219) (size 0.8) (drill 0.4) (layers F.Cu B.Cu) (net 16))
 (segment (start 86.36 101.219) (end 81.28 101.219) (width 0.25) (layer B.Cu) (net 16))
 (segment (start 81.28 101.219) (end 80.518 101.981) (width 0.25) (layer B.Cu) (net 16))
 (segment (start 80.518 101.981) (end 80.518 106.3625) (width 0.25) (layer B.Cu) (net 16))
 (segment (start 80.518 106.3625) (end 80.772 106.6165) (width 0.25) (layer B.Cu) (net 16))
 (segment (start 80.772 106.6165) (end 84.328 106.6165) (width 0.25) (layer B.Cu) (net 16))
 (segment (start 84.328 106.6165) (end 84.582 106.8705) (width 0.25) (layer B.Cu) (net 16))
 (segment (start 84.582 106.8705) (end 84.582 109.0295) (width 0.25) (layer B.Cu) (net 16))
 (segment (start 84.582 109.0295) (end 84.963 109.4105) (width 0.25) (layer B.Cu) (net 16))
 (segment (start 84.963 109.4105) (end 89.3445 109.4105) (width 0.25) (layer B.Cu) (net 16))
 (segment (start 90.678 108.077) (end 92.71 108.077) (width 0.25) (layer B.Cu) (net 16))
 (segment (start 89.3445 109.4105) (end 90.678 108.077) (width 0.25) (layer B.Cu) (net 16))
 (segment (start 83.747001 98.280999) (end 83.182 98.846) (width 0.25) (layer F.Cu) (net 15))
 (segment (start 83.182 98.846) (end 83.182 98.8665) (width 0.25) (layer F.Cu) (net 15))
 (segment (start 85.715 102.455) (end 84.421 102.455) (width 0.25) (layer F.Cu) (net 15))
 (segment (start 84.421 102.455) (end 84.2645 102.2985) (width 0.25) (layer F.Cu) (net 15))
 (segment (start 84.2645 99.9285) (end 83.182 98.846) (width 0.25) (layer F.Cu) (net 15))
 (segment (start 84.2645 102.2985) (end 84.2645 99.9285) (width 0.25) (layer F.Cu) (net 15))
 (segment (start 83.172 101.506) (end 83.172 102.2855) (width 0.25) (layer F.Cu) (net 14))
 (segment (start 84.6115 103.725) (end 85.715 103.725) (width 0.25) (layer F.Cu) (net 14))
 (segment (start 83.172 102.2855) (end 84.6115 103.725) (width 0.25) (layer F.Cu) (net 14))
 (segment (start 84.74 104.995) (end 85.715 104.995) (width 0.25) (layer F.Cu) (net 13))
 (segment (start 85.715 104.995) (end 84.548 104.995) (width 0.25) (layer F.Cu) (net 13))
 (segment (start 84.139 104.586) (end 83.142 104.586) (width 0.25) (layer F.Cu) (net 13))
 (segment (start 84.548 104.995) (end 84.139 104.586) (width 0.25) (layer F.Cu) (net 13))
 (segment (start 84.74 106.265) (end 85.715 106.265) (width 0.25) (layer F.Cu) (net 12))
 (segment (start 83.122 107.526) (end 83.122 106.87) (width 0.25) (layer F.Cu) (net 12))
 (segment (start 83.727 106.265) (end 85.715 106.265) (width 0.25) (layer F.Cu) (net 12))
 (segment (start 83.122 106.87) (end 83.727 106.265) (width 0.25) (layer F.Cu) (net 12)))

